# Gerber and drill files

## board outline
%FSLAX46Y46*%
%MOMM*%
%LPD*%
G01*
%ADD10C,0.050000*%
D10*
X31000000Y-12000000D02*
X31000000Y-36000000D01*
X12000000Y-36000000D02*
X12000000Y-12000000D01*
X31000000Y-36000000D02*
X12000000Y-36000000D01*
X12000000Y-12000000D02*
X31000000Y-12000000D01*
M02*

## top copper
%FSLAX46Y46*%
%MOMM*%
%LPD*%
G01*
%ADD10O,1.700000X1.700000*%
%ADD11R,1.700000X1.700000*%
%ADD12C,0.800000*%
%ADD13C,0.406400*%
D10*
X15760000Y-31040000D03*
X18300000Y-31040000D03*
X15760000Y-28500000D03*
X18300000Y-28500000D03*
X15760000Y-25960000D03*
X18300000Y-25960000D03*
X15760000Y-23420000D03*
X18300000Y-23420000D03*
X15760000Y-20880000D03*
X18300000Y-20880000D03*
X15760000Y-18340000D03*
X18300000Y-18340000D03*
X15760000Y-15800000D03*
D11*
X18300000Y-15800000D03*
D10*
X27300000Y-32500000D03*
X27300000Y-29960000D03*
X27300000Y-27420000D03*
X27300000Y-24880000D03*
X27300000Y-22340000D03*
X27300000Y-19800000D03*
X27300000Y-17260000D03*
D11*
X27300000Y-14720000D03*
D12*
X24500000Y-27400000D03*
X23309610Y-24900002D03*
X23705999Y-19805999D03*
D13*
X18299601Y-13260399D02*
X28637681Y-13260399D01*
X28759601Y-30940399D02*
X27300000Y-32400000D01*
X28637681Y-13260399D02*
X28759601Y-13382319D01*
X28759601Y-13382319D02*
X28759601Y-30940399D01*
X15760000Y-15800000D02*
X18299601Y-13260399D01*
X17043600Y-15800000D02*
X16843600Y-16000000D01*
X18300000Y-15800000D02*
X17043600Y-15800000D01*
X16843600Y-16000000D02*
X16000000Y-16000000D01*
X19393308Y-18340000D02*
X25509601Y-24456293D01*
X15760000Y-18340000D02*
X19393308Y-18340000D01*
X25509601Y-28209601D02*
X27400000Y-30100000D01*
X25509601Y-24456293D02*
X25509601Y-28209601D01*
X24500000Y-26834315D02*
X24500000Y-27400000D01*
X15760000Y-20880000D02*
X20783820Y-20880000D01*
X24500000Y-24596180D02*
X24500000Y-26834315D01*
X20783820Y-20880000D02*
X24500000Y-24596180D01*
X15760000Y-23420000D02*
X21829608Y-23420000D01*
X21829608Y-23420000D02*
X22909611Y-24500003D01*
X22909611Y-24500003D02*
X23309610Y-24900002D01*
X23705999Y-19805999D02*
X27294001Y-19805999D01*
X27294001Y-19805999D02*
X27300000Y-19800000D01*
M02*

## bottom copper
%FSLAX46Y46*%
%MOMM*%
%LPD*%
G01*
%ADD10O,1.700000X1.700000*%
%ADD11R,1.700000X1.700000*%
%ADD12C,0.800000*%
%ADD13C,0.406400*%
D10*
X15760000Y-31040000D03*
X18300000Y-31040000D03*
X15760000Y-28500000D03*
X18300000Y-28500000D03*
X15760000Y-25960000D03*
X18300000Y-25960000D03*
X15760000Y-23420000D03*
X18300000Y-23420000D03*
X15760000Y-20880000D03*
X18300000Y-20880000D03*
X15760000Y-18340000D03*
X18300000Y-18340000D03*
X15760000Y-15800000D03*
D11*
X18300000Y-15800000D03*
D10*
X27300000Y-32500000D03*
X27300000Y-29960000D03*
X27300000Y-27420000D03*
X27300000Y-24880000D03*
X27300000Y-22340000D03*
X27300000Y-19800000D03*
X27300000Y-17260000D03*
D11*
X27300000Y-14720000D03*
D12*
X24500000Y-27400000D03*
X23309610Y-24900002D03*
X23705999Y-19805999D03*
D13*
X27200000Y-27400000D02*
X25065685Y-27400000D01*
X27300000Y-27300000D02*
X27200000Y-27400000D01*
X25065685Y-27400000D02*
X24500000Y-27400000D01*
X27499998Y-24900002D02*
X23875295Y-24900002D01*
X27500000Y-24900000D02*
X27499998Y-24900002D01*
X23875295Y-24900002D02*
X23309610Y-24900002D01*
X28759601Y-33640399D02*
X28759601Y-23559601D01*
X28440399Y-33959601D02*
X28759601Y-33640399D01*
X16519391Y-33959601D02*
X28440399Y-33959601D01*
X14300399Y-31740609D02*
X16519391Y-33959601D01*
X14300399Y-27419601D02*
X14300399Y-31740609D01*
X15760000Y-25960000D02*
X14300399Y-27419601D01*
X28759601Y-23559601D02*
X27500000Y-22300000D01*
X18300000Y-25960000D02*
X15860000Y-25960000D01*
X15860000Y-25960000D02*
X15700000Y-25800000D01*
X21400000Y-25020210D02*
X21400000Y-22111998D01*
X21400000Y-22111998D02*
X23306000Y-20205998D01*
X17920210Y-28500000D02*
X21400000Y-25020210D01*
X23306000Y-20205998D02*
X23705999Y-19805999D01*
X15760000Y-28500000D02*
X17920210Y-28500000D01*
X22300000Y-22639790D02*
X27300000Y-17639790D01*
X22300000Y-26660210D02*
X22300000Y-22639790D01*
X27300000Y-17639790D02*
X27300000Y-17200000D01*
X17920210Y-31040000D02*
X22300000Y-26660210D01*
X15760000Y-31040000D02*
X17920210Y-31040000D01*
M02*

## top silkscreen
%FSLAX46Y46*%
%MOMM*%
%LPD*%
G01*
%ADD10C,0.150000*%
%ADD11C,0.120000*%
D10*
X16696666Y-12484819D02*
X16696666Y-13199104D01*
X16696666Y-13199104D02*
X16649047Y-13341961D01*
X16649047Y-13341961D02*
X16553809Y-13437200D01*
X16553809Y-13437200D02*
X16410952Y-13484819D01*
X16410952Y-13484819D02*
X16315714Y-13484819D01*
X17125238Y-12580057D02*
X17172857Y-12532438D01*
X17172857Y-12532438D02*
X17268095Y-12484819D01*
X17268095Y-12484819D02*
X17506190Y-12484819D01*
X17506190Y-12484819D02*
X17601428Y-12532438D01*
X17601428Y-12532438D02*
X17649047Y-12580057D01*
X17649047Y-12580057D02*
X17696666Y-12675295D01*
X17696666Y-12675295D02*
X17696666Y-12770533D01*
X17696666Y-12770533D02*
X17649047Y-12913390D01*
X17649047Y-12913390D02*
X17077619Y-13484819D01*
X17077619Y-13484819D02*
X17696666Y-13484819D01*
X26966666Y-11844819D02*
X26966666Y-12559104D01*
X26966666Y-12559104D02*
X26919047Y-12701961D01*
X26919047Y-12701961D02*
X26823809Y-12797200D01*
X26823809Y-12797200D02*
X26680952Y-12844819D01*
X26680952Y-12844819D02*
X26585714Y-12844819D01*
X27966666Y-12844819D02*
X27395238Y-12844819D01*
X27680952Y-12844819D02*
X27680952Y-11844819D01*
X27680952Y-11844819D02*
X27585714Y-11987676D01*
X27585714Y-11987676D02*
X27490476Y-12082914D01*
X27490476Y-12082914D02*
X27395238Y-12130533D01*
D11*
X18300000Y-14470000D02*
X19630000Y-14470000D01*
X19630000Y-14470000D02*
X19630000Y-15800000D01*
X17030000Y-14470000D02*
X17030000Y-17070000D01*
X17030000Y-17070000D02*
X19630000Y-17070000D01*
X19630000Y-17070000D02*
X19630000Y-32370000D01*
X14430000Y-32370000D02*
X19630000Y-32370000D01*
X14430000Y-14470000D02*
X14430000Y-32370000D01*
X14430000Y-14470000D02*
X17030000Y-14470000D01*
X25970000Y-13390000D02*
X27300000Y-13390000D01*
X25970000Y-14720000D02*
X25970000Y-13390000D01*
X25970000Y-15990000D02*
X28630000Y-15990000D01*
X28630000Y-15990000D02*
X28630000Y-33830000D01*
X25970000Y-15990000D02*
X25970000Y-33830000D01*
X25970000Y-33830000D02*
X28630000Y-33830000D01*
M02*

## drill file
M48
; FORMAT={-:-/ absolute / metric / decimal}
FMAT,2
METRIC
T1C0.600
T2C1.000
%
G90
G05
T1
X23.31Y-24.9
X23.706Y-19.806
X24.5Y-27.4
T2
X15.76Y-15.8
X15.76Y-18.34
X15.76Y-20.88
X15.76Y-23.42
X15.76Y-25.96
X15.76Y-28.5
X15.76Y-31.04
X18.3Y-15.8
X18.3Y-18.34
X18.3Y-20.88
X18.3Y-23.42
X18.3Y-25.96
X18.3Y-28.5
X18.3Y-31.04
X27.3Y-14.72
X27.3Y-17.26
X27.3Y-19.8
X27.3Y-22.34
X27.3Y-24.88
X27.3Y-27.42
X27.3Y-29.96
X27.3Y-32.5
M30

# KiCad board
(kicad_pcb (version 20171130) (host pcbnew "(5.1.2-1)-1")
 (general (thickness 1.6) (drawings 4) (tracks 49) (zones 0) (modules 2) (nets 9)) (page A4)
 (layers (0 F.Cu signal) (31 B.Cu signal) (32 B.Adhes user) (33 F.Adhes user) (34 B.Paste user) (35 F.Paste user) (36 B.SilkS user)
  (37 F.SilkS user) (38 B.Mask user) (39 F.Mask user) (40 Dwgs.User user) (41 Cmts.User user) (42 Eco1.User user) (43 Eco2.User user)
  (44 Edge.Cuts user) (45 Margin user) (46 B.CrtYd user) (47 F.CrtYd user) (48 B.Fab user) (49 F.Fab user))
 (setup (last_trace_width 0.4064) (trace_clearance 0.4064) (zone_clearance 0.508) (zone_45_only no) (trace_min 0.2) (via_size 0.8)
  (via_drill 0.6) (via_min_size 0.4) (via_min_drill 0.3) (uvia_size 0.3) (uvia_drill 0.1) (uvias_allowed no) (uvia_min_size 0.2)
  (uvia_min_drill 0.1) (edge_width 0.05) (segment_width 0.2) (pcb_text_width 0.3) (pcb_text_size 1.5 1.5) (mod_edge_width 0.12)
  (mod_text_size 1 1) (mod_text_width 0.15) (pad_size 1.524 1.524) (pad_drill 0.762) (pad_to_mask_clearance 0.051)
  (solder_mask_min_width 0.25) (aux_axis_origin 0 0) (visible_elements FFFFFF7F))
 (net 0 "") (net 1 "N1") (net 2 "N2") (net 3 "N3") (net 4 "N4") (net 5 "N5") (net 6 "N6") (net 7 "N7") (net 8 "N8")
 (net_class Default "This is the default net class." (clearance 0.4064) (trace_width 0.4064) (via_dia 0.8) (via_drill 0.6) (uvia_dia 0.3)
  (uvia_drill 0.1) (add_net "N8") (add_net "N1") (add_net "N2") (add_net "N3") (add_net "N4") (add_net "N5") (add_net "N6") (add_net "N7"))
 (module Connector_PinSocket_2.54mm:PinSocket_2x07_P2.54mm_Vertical (layer F.Cu) (at 18.3 15.8)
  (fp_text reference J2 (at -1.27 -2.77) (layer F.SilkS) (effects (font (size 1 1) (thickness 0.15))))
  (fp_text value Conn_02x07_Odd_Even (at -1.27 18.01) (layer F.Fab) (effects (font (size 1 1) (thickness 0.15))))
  (fp_line (start 0 -1.33) (end 1.33 -1.33) (layer F.SilkS) (width 0.12))
  (fp_line (start 1.33 -1.33) (end 1.33 0) (layer F.SilkS) (width 0.12))
  (fp_line (start -1.27 -1.33) (end -1.27 1.27) (layer F.SilkS) (width 0.12))
  (fp_line (start -1.27 1.27) (end 1.33 1.27) (layer F.SilkS) (width 0.12))
  (fp_line (start 1.33 1.27) (end 1.33 16.57) (layer F.SilkS) (width 0.12))
  (fp_line (start -3.87 16.57) (end 1.33 16.57) (layer F.SilkS) (width 0.12))
  (fp_line (start -3.87 -1.33) (end -3.87 16.57) (layer F.SilkS) (width 0.12))
  (fp_line (start -3.87 -1.33) (end -1.27 -1.33) (layer F.SilkS) (width 0.12))
  (pad 14 thru_hole oval (at -2.54 15.24) (size 1.7 1.7) (drill 1) (layers *.Cu *.Mask) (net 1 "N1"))
  (pad 13 thru_hole oval (at 0 15.24) (size 1.7 1.7) (drill 1) (layers *.Cu *.Mask) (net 1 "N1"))
  (pad 12 thru_hole oval (at -2.54 12.7) (size 1.7 1.7) (drill 1) (layers *.Cu *.Mask) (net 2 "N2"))
  (pad 11 thru_hole oval (at 0 12.7) (size 1.7 1.7) (drill 1) (layers *.Cu *.Mask) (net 2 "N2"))
  (pad 10 thru_hole oval (at -2.54 10.16) (size 1.7 1.7) (drill 1) (layers *.Cu *.Mask) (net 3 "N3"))
  (pad 9 thru_hole oval (at 0 10.16) (size 1.7 1.7) (drill 1) (layers *.Cu *.Mask) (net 3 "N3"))
  (pad 8 thru_hole oval (at -2.54 7.62) (size 1.7 1.7) (drill 1) (layers *.Cu *.Mask) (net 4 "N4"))
  (pad 7 thru_hole oval (at 0 7.62) (size 1.7 1.7) (drill 1) (layers *.Cu *.Mask) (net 4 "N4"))
  (pad 6 thru_hole oval (at -2.54 5.08) (size 1.7 1.7) (drill 1) (layers *.Cu *.Mask) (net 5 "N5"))
  (pad 5 thru_hole oval (at 0 5.08) (size 1.7 1.7) (drill 1) (layers *.Cu *.Mask) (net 5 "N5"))
  (pad 4 thru_hole oval (at -2.54 2.54) (size 1.7 1.7) (drill 1) (layers *.Cu *.Mask) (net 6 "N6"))
  (pad 3 thru_hole oval (at 0 2.54) (size 1.7 1.7) (drill 1) (layers *.Cu *.Mask) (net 6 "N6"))
  (pad 2 thru_hole oval (at -2.54 0) (size 1.7 1.7) (drill 1) (layers *.Cu *.Mask) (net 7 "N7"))
  (pad 1 thru_hole rect (at 0 0) (size 1.7 1.7) (drill 1) (layers *.Cu *.Mask) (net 7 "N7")))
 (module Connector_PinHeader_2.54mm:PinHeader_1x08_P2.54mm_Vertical (layer F.Cu) (at 27.3 14.72)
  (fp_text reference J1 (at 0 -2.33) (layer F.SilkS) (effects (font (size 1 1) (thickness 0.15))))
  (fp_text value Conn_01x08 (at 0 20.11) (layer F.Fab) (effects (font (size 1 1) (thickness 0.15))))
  (fp_line (start -1.33 -1.33) (end 0 -1.33) (layer F.SilkS) (width 0.12))
  (fp_line (start -1.33 0) (end -1.33 -1.33) (layer F.SilkS) (width 0.12))
  (fp_line (start -1.33 1.27) (end 1.33 1.27) (layer F.SilkS) (width 0.12))
  (fp_line (start 1.33 1.27) (end 1.33 19.11) (layer F.SilkS) (width 0.12))
  (fp_line (start -1.33 1.27) (end -1.33 19.11) (layer F.SilkS) (width 0.12))
  (fp_line (start -1.33 19.11) (end 1.33 19.11) (layer F.SilkS) (width 0.12))
  (pad 8 thru_hole oval (at 0 17.78) (size 1.7 1.7) (drill 1) (layers *.Cu *.Mask) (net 7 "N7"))
  (pad 7 thru_hole oval (at 0 15.24) (size 1.7 1.7) (drill 1) (layers *.Cu *.Mask) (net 6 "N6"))
  (pad 6 thru_hole oval (at 0 12.7) (size 1.7 1.7) (drill 1) (layers *.Cu *.Mask) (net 5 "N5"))
  (pad 5 thru_hole oval (at 0 10.16) (size 1.7 1.7) (drill 1) (layers *.Cu *.Mask) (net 4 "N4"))
  (pad 4 thru_hole oval (at 0 7.62) (size 1.7 1.7) (drill 1) (layers *.Cu *.Mask) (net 3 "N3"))
  (pad 3 thru_hole oval (at 0 5.08) (size 1.7 1.7) (drill 1) (layers *.Cu *.Mask) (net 2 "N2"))
  (pad 2 thru_hole oval (at 0 2.54) (size 1.7 1.7) (drill 1) (layers *.Cu *.Mask) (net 1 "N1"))
  (pad 1 thru_hole rect (at 0 0) (size 1.7 1.7) (drill 1) (layers *.Cu *.Mask) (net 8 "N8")))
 (gr_line (start 31 12) (end 31 36) (layer Edge.Cuts) (width 0.05))
 (gr_line (start 12 36) (end 12 12) (layer Edge.Cuts) (width 0.05))
 (gr_line (start 31 36) (end 12 36) (layer Edge.Cuts) (width 0.05))
 (gr_line (start 12 12) (end 31 12) (layer Edge.Cuts) (width 0.05))
 (segment (start 18.299601 13.260399) (end 28.637681 13.260399) (width 0.4064) (layer F.Cu) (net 7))
 (segment (start 28.759601 30.940399) (end 27.3 32.4) (width 0.4064) (layer F.Cu) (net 7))
 (segment (start 28.637681 13.260399) (end 28.759601 13.382319) (width 0.4064) (layer F.Cu) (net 7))
 (segment (start 28.759601 13.382319) (end 28.759601 30.940399) (width 0.4064) (layer F.Cu) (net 7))
 (segment (start 15.76 15.8) (end 18.299601 13.260399) (width 0.4064) (layer F.Cu) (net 7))
 (segment (start 17.0436 15.8) (end 16.8436 16) (width 0.4064) (layer F.Cu) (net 7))
 (segment (start 18.3 15.8) (end 17.0436 15.8) (width 0.4064) (layer F.Cu) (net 7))
 (segment (start 16.8436 16) (end 16 16) (width 0.4064) (layer F.Cu) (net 7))
 (segment (start 19.393308 18.34) (end 25.509601 24.456293) (width 0.4064) (layer F.Cu) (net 6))
 (segment (start 15.76 18.34) (end 19.393308 18.34) (width 0.4064) (layer F.Cu) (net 6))
 (segment (start 25.509601 28.209601) (end 27.4 30.1) (width 0.4064) (layer F.Cu) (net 6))
 (segment (start 25.509601 24.456293) (end 25.509601 28.209601) (width 0.4064) (layer F.Cu) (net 6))
 (segment (start 27.2 27.4) (end 25.065685 27.4) (width 0.4064) (layer B.Cu) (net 5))
 (via (at 24.5 27.4) (size 0.8) (drill 0.6) (layers F.Cu B.Cu) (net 5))
 (segment (start 27.3 27.3) (end 27.2 27.4) (width 0.4064) (layer B.Cu) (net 5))
 (segment (start 25.065685 27.4) (end 24.5 27.4) (width 0.4064) (layer B.Cu) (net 5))
 (segment (start 24.5 26.834315) (end 24.5 27.4) (width 0.4064) (layer F.Cu) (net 5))
 (segment (start 15.76 20.88) (end 20.78382 20.88) (width 0.4064) (layer F.Cu) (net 5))
 (segment (start 24.5 24.59618) (end 24.5 26.834315) (width 0.4064) (layer F.Cu) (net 5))
 (segment (start 20.78382 20.88) (end 24.5 24.59618) (width 0.4064) (layer F.Cu) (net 5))
 (via (at 23.30961 24.900002) (size 0.8) (drill 0.6) (layers F.Cu B.Cu) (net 4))
 (segment (start 27.499998 24.900002) (end 23.875295 24.900002) (width 0.4064) (layer B.Cu) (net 4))
 (segment (start 27.5 24.9) (end 27.499998 24.900002) (width 0.4064) (layer B.Cu) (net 4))
 (segment (start 15.76 23.42) (end 21.829608 23.42) (width 0.4064) (layer F.Cu) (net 4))
 (segment (start 21.829608 23.42) (end 22.909611 24.500003) (width 0.4064) (layer F.Cu) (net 4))
 (segment (start 23.875295 24.900002) (end 23.30961 24.900002) (width 0.4064) (layer B.Cu) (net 4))
 (segment (start 22.909611 24.500003) (end 23.30961 24.900002) (width 0.4064) (layer F.Cu) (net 4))
 (segment (start 28.759601 33.640399) (end 28.759601 23.559601) (width 0.4064) (layer B.Cu) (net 3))
 (segment (start 28.440399 33.959601) (end 28.759601 33.640399) (width 0.4064) (layer B.Cu) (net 3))
 (segment (start 16.519391 33.959601) (end 28.440399 33.959601) (width 0.4064) (layer B.Cu) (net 3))
 (segment (start 14.300399 31.740609) (end 16.519391 33.959601) (width 0.4064) (layer B.Cu) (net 3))
 (segment (start 14.300399 27.419601) (end 14.300399 31.740609) (width 0.4064) (layer B.Cu) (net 3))
 (segment (start 15.76 25.96) (end 14.300399 27.419601) (width 0.4064) (layer B.Cu) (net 3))
 (segment (start 28.759601 23.559601) (end 27.5 22.3) (width 0.4064) (layer B.Cu) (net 3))
 (segment (start 18.3 25.96) (end 15.86 25.96) (width 0.4064) (layer B.Cu) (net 3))
 (segment (start 15.86 25.96) (end 15.7 25.8) (width 0.4064) (layer B.Cu) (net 3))
 (via (at 23.705999 19.805999) (size 0.8) (drill 0.6) (layers F.Cu B.Cu) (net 2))
 (segment (start 23.705999 19.805999) (end 27.294001 19.805999) (width 0.4064) (layer F.Cu) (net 2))
 (segment (start 27.294001 19.805999) (end 27.3 19.8) (width 0.4064) (layer F.Cu) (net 2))
 (segment (start 21.4 25.02021) (end 21.4 22.111998) (width 0.4064) (layer B.Cu) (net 2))
 (segment (start 21.4 22.111998) (end 23.306 20.205998) (width 0.4064) (layer B.Cu) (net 2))
 (segment (start 17.92021 28.5) (end 21.4 25.02021) (width 0.4064) (layer B.Cu) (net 2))
 (segment (start 23.306 20.205998) (end 23.705999 19.805999) (width 0.4064) (layer B.Cu) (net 2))
 (segment (start 15.76 28.5) (end 17.92021 28.5) (width 0.4064) (layer B.Cu) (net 2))
 (segment (start 22.3 22.63979) (end 27.3 17.63979) (width 0.4064) (layer B.Cu) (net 1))
 (segment (start 22.3 26.66021) (end 22.3 22.63979) (width 0.4064) (layer B.Cu) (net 1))
 (segment (start 27.3 17.63979) (end 27.3 17.2) (width 0.4064) (layer B.Cu) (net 1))
 (segment (start 17.92021 31.04) (end 22.3 26.66021) (width 0.4064) (layer B.Cu) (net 1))
 (segment (start 15.76 31.04) (end 17.92021 31.04) (width 0.4064) (layer B.Cu) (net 1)))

